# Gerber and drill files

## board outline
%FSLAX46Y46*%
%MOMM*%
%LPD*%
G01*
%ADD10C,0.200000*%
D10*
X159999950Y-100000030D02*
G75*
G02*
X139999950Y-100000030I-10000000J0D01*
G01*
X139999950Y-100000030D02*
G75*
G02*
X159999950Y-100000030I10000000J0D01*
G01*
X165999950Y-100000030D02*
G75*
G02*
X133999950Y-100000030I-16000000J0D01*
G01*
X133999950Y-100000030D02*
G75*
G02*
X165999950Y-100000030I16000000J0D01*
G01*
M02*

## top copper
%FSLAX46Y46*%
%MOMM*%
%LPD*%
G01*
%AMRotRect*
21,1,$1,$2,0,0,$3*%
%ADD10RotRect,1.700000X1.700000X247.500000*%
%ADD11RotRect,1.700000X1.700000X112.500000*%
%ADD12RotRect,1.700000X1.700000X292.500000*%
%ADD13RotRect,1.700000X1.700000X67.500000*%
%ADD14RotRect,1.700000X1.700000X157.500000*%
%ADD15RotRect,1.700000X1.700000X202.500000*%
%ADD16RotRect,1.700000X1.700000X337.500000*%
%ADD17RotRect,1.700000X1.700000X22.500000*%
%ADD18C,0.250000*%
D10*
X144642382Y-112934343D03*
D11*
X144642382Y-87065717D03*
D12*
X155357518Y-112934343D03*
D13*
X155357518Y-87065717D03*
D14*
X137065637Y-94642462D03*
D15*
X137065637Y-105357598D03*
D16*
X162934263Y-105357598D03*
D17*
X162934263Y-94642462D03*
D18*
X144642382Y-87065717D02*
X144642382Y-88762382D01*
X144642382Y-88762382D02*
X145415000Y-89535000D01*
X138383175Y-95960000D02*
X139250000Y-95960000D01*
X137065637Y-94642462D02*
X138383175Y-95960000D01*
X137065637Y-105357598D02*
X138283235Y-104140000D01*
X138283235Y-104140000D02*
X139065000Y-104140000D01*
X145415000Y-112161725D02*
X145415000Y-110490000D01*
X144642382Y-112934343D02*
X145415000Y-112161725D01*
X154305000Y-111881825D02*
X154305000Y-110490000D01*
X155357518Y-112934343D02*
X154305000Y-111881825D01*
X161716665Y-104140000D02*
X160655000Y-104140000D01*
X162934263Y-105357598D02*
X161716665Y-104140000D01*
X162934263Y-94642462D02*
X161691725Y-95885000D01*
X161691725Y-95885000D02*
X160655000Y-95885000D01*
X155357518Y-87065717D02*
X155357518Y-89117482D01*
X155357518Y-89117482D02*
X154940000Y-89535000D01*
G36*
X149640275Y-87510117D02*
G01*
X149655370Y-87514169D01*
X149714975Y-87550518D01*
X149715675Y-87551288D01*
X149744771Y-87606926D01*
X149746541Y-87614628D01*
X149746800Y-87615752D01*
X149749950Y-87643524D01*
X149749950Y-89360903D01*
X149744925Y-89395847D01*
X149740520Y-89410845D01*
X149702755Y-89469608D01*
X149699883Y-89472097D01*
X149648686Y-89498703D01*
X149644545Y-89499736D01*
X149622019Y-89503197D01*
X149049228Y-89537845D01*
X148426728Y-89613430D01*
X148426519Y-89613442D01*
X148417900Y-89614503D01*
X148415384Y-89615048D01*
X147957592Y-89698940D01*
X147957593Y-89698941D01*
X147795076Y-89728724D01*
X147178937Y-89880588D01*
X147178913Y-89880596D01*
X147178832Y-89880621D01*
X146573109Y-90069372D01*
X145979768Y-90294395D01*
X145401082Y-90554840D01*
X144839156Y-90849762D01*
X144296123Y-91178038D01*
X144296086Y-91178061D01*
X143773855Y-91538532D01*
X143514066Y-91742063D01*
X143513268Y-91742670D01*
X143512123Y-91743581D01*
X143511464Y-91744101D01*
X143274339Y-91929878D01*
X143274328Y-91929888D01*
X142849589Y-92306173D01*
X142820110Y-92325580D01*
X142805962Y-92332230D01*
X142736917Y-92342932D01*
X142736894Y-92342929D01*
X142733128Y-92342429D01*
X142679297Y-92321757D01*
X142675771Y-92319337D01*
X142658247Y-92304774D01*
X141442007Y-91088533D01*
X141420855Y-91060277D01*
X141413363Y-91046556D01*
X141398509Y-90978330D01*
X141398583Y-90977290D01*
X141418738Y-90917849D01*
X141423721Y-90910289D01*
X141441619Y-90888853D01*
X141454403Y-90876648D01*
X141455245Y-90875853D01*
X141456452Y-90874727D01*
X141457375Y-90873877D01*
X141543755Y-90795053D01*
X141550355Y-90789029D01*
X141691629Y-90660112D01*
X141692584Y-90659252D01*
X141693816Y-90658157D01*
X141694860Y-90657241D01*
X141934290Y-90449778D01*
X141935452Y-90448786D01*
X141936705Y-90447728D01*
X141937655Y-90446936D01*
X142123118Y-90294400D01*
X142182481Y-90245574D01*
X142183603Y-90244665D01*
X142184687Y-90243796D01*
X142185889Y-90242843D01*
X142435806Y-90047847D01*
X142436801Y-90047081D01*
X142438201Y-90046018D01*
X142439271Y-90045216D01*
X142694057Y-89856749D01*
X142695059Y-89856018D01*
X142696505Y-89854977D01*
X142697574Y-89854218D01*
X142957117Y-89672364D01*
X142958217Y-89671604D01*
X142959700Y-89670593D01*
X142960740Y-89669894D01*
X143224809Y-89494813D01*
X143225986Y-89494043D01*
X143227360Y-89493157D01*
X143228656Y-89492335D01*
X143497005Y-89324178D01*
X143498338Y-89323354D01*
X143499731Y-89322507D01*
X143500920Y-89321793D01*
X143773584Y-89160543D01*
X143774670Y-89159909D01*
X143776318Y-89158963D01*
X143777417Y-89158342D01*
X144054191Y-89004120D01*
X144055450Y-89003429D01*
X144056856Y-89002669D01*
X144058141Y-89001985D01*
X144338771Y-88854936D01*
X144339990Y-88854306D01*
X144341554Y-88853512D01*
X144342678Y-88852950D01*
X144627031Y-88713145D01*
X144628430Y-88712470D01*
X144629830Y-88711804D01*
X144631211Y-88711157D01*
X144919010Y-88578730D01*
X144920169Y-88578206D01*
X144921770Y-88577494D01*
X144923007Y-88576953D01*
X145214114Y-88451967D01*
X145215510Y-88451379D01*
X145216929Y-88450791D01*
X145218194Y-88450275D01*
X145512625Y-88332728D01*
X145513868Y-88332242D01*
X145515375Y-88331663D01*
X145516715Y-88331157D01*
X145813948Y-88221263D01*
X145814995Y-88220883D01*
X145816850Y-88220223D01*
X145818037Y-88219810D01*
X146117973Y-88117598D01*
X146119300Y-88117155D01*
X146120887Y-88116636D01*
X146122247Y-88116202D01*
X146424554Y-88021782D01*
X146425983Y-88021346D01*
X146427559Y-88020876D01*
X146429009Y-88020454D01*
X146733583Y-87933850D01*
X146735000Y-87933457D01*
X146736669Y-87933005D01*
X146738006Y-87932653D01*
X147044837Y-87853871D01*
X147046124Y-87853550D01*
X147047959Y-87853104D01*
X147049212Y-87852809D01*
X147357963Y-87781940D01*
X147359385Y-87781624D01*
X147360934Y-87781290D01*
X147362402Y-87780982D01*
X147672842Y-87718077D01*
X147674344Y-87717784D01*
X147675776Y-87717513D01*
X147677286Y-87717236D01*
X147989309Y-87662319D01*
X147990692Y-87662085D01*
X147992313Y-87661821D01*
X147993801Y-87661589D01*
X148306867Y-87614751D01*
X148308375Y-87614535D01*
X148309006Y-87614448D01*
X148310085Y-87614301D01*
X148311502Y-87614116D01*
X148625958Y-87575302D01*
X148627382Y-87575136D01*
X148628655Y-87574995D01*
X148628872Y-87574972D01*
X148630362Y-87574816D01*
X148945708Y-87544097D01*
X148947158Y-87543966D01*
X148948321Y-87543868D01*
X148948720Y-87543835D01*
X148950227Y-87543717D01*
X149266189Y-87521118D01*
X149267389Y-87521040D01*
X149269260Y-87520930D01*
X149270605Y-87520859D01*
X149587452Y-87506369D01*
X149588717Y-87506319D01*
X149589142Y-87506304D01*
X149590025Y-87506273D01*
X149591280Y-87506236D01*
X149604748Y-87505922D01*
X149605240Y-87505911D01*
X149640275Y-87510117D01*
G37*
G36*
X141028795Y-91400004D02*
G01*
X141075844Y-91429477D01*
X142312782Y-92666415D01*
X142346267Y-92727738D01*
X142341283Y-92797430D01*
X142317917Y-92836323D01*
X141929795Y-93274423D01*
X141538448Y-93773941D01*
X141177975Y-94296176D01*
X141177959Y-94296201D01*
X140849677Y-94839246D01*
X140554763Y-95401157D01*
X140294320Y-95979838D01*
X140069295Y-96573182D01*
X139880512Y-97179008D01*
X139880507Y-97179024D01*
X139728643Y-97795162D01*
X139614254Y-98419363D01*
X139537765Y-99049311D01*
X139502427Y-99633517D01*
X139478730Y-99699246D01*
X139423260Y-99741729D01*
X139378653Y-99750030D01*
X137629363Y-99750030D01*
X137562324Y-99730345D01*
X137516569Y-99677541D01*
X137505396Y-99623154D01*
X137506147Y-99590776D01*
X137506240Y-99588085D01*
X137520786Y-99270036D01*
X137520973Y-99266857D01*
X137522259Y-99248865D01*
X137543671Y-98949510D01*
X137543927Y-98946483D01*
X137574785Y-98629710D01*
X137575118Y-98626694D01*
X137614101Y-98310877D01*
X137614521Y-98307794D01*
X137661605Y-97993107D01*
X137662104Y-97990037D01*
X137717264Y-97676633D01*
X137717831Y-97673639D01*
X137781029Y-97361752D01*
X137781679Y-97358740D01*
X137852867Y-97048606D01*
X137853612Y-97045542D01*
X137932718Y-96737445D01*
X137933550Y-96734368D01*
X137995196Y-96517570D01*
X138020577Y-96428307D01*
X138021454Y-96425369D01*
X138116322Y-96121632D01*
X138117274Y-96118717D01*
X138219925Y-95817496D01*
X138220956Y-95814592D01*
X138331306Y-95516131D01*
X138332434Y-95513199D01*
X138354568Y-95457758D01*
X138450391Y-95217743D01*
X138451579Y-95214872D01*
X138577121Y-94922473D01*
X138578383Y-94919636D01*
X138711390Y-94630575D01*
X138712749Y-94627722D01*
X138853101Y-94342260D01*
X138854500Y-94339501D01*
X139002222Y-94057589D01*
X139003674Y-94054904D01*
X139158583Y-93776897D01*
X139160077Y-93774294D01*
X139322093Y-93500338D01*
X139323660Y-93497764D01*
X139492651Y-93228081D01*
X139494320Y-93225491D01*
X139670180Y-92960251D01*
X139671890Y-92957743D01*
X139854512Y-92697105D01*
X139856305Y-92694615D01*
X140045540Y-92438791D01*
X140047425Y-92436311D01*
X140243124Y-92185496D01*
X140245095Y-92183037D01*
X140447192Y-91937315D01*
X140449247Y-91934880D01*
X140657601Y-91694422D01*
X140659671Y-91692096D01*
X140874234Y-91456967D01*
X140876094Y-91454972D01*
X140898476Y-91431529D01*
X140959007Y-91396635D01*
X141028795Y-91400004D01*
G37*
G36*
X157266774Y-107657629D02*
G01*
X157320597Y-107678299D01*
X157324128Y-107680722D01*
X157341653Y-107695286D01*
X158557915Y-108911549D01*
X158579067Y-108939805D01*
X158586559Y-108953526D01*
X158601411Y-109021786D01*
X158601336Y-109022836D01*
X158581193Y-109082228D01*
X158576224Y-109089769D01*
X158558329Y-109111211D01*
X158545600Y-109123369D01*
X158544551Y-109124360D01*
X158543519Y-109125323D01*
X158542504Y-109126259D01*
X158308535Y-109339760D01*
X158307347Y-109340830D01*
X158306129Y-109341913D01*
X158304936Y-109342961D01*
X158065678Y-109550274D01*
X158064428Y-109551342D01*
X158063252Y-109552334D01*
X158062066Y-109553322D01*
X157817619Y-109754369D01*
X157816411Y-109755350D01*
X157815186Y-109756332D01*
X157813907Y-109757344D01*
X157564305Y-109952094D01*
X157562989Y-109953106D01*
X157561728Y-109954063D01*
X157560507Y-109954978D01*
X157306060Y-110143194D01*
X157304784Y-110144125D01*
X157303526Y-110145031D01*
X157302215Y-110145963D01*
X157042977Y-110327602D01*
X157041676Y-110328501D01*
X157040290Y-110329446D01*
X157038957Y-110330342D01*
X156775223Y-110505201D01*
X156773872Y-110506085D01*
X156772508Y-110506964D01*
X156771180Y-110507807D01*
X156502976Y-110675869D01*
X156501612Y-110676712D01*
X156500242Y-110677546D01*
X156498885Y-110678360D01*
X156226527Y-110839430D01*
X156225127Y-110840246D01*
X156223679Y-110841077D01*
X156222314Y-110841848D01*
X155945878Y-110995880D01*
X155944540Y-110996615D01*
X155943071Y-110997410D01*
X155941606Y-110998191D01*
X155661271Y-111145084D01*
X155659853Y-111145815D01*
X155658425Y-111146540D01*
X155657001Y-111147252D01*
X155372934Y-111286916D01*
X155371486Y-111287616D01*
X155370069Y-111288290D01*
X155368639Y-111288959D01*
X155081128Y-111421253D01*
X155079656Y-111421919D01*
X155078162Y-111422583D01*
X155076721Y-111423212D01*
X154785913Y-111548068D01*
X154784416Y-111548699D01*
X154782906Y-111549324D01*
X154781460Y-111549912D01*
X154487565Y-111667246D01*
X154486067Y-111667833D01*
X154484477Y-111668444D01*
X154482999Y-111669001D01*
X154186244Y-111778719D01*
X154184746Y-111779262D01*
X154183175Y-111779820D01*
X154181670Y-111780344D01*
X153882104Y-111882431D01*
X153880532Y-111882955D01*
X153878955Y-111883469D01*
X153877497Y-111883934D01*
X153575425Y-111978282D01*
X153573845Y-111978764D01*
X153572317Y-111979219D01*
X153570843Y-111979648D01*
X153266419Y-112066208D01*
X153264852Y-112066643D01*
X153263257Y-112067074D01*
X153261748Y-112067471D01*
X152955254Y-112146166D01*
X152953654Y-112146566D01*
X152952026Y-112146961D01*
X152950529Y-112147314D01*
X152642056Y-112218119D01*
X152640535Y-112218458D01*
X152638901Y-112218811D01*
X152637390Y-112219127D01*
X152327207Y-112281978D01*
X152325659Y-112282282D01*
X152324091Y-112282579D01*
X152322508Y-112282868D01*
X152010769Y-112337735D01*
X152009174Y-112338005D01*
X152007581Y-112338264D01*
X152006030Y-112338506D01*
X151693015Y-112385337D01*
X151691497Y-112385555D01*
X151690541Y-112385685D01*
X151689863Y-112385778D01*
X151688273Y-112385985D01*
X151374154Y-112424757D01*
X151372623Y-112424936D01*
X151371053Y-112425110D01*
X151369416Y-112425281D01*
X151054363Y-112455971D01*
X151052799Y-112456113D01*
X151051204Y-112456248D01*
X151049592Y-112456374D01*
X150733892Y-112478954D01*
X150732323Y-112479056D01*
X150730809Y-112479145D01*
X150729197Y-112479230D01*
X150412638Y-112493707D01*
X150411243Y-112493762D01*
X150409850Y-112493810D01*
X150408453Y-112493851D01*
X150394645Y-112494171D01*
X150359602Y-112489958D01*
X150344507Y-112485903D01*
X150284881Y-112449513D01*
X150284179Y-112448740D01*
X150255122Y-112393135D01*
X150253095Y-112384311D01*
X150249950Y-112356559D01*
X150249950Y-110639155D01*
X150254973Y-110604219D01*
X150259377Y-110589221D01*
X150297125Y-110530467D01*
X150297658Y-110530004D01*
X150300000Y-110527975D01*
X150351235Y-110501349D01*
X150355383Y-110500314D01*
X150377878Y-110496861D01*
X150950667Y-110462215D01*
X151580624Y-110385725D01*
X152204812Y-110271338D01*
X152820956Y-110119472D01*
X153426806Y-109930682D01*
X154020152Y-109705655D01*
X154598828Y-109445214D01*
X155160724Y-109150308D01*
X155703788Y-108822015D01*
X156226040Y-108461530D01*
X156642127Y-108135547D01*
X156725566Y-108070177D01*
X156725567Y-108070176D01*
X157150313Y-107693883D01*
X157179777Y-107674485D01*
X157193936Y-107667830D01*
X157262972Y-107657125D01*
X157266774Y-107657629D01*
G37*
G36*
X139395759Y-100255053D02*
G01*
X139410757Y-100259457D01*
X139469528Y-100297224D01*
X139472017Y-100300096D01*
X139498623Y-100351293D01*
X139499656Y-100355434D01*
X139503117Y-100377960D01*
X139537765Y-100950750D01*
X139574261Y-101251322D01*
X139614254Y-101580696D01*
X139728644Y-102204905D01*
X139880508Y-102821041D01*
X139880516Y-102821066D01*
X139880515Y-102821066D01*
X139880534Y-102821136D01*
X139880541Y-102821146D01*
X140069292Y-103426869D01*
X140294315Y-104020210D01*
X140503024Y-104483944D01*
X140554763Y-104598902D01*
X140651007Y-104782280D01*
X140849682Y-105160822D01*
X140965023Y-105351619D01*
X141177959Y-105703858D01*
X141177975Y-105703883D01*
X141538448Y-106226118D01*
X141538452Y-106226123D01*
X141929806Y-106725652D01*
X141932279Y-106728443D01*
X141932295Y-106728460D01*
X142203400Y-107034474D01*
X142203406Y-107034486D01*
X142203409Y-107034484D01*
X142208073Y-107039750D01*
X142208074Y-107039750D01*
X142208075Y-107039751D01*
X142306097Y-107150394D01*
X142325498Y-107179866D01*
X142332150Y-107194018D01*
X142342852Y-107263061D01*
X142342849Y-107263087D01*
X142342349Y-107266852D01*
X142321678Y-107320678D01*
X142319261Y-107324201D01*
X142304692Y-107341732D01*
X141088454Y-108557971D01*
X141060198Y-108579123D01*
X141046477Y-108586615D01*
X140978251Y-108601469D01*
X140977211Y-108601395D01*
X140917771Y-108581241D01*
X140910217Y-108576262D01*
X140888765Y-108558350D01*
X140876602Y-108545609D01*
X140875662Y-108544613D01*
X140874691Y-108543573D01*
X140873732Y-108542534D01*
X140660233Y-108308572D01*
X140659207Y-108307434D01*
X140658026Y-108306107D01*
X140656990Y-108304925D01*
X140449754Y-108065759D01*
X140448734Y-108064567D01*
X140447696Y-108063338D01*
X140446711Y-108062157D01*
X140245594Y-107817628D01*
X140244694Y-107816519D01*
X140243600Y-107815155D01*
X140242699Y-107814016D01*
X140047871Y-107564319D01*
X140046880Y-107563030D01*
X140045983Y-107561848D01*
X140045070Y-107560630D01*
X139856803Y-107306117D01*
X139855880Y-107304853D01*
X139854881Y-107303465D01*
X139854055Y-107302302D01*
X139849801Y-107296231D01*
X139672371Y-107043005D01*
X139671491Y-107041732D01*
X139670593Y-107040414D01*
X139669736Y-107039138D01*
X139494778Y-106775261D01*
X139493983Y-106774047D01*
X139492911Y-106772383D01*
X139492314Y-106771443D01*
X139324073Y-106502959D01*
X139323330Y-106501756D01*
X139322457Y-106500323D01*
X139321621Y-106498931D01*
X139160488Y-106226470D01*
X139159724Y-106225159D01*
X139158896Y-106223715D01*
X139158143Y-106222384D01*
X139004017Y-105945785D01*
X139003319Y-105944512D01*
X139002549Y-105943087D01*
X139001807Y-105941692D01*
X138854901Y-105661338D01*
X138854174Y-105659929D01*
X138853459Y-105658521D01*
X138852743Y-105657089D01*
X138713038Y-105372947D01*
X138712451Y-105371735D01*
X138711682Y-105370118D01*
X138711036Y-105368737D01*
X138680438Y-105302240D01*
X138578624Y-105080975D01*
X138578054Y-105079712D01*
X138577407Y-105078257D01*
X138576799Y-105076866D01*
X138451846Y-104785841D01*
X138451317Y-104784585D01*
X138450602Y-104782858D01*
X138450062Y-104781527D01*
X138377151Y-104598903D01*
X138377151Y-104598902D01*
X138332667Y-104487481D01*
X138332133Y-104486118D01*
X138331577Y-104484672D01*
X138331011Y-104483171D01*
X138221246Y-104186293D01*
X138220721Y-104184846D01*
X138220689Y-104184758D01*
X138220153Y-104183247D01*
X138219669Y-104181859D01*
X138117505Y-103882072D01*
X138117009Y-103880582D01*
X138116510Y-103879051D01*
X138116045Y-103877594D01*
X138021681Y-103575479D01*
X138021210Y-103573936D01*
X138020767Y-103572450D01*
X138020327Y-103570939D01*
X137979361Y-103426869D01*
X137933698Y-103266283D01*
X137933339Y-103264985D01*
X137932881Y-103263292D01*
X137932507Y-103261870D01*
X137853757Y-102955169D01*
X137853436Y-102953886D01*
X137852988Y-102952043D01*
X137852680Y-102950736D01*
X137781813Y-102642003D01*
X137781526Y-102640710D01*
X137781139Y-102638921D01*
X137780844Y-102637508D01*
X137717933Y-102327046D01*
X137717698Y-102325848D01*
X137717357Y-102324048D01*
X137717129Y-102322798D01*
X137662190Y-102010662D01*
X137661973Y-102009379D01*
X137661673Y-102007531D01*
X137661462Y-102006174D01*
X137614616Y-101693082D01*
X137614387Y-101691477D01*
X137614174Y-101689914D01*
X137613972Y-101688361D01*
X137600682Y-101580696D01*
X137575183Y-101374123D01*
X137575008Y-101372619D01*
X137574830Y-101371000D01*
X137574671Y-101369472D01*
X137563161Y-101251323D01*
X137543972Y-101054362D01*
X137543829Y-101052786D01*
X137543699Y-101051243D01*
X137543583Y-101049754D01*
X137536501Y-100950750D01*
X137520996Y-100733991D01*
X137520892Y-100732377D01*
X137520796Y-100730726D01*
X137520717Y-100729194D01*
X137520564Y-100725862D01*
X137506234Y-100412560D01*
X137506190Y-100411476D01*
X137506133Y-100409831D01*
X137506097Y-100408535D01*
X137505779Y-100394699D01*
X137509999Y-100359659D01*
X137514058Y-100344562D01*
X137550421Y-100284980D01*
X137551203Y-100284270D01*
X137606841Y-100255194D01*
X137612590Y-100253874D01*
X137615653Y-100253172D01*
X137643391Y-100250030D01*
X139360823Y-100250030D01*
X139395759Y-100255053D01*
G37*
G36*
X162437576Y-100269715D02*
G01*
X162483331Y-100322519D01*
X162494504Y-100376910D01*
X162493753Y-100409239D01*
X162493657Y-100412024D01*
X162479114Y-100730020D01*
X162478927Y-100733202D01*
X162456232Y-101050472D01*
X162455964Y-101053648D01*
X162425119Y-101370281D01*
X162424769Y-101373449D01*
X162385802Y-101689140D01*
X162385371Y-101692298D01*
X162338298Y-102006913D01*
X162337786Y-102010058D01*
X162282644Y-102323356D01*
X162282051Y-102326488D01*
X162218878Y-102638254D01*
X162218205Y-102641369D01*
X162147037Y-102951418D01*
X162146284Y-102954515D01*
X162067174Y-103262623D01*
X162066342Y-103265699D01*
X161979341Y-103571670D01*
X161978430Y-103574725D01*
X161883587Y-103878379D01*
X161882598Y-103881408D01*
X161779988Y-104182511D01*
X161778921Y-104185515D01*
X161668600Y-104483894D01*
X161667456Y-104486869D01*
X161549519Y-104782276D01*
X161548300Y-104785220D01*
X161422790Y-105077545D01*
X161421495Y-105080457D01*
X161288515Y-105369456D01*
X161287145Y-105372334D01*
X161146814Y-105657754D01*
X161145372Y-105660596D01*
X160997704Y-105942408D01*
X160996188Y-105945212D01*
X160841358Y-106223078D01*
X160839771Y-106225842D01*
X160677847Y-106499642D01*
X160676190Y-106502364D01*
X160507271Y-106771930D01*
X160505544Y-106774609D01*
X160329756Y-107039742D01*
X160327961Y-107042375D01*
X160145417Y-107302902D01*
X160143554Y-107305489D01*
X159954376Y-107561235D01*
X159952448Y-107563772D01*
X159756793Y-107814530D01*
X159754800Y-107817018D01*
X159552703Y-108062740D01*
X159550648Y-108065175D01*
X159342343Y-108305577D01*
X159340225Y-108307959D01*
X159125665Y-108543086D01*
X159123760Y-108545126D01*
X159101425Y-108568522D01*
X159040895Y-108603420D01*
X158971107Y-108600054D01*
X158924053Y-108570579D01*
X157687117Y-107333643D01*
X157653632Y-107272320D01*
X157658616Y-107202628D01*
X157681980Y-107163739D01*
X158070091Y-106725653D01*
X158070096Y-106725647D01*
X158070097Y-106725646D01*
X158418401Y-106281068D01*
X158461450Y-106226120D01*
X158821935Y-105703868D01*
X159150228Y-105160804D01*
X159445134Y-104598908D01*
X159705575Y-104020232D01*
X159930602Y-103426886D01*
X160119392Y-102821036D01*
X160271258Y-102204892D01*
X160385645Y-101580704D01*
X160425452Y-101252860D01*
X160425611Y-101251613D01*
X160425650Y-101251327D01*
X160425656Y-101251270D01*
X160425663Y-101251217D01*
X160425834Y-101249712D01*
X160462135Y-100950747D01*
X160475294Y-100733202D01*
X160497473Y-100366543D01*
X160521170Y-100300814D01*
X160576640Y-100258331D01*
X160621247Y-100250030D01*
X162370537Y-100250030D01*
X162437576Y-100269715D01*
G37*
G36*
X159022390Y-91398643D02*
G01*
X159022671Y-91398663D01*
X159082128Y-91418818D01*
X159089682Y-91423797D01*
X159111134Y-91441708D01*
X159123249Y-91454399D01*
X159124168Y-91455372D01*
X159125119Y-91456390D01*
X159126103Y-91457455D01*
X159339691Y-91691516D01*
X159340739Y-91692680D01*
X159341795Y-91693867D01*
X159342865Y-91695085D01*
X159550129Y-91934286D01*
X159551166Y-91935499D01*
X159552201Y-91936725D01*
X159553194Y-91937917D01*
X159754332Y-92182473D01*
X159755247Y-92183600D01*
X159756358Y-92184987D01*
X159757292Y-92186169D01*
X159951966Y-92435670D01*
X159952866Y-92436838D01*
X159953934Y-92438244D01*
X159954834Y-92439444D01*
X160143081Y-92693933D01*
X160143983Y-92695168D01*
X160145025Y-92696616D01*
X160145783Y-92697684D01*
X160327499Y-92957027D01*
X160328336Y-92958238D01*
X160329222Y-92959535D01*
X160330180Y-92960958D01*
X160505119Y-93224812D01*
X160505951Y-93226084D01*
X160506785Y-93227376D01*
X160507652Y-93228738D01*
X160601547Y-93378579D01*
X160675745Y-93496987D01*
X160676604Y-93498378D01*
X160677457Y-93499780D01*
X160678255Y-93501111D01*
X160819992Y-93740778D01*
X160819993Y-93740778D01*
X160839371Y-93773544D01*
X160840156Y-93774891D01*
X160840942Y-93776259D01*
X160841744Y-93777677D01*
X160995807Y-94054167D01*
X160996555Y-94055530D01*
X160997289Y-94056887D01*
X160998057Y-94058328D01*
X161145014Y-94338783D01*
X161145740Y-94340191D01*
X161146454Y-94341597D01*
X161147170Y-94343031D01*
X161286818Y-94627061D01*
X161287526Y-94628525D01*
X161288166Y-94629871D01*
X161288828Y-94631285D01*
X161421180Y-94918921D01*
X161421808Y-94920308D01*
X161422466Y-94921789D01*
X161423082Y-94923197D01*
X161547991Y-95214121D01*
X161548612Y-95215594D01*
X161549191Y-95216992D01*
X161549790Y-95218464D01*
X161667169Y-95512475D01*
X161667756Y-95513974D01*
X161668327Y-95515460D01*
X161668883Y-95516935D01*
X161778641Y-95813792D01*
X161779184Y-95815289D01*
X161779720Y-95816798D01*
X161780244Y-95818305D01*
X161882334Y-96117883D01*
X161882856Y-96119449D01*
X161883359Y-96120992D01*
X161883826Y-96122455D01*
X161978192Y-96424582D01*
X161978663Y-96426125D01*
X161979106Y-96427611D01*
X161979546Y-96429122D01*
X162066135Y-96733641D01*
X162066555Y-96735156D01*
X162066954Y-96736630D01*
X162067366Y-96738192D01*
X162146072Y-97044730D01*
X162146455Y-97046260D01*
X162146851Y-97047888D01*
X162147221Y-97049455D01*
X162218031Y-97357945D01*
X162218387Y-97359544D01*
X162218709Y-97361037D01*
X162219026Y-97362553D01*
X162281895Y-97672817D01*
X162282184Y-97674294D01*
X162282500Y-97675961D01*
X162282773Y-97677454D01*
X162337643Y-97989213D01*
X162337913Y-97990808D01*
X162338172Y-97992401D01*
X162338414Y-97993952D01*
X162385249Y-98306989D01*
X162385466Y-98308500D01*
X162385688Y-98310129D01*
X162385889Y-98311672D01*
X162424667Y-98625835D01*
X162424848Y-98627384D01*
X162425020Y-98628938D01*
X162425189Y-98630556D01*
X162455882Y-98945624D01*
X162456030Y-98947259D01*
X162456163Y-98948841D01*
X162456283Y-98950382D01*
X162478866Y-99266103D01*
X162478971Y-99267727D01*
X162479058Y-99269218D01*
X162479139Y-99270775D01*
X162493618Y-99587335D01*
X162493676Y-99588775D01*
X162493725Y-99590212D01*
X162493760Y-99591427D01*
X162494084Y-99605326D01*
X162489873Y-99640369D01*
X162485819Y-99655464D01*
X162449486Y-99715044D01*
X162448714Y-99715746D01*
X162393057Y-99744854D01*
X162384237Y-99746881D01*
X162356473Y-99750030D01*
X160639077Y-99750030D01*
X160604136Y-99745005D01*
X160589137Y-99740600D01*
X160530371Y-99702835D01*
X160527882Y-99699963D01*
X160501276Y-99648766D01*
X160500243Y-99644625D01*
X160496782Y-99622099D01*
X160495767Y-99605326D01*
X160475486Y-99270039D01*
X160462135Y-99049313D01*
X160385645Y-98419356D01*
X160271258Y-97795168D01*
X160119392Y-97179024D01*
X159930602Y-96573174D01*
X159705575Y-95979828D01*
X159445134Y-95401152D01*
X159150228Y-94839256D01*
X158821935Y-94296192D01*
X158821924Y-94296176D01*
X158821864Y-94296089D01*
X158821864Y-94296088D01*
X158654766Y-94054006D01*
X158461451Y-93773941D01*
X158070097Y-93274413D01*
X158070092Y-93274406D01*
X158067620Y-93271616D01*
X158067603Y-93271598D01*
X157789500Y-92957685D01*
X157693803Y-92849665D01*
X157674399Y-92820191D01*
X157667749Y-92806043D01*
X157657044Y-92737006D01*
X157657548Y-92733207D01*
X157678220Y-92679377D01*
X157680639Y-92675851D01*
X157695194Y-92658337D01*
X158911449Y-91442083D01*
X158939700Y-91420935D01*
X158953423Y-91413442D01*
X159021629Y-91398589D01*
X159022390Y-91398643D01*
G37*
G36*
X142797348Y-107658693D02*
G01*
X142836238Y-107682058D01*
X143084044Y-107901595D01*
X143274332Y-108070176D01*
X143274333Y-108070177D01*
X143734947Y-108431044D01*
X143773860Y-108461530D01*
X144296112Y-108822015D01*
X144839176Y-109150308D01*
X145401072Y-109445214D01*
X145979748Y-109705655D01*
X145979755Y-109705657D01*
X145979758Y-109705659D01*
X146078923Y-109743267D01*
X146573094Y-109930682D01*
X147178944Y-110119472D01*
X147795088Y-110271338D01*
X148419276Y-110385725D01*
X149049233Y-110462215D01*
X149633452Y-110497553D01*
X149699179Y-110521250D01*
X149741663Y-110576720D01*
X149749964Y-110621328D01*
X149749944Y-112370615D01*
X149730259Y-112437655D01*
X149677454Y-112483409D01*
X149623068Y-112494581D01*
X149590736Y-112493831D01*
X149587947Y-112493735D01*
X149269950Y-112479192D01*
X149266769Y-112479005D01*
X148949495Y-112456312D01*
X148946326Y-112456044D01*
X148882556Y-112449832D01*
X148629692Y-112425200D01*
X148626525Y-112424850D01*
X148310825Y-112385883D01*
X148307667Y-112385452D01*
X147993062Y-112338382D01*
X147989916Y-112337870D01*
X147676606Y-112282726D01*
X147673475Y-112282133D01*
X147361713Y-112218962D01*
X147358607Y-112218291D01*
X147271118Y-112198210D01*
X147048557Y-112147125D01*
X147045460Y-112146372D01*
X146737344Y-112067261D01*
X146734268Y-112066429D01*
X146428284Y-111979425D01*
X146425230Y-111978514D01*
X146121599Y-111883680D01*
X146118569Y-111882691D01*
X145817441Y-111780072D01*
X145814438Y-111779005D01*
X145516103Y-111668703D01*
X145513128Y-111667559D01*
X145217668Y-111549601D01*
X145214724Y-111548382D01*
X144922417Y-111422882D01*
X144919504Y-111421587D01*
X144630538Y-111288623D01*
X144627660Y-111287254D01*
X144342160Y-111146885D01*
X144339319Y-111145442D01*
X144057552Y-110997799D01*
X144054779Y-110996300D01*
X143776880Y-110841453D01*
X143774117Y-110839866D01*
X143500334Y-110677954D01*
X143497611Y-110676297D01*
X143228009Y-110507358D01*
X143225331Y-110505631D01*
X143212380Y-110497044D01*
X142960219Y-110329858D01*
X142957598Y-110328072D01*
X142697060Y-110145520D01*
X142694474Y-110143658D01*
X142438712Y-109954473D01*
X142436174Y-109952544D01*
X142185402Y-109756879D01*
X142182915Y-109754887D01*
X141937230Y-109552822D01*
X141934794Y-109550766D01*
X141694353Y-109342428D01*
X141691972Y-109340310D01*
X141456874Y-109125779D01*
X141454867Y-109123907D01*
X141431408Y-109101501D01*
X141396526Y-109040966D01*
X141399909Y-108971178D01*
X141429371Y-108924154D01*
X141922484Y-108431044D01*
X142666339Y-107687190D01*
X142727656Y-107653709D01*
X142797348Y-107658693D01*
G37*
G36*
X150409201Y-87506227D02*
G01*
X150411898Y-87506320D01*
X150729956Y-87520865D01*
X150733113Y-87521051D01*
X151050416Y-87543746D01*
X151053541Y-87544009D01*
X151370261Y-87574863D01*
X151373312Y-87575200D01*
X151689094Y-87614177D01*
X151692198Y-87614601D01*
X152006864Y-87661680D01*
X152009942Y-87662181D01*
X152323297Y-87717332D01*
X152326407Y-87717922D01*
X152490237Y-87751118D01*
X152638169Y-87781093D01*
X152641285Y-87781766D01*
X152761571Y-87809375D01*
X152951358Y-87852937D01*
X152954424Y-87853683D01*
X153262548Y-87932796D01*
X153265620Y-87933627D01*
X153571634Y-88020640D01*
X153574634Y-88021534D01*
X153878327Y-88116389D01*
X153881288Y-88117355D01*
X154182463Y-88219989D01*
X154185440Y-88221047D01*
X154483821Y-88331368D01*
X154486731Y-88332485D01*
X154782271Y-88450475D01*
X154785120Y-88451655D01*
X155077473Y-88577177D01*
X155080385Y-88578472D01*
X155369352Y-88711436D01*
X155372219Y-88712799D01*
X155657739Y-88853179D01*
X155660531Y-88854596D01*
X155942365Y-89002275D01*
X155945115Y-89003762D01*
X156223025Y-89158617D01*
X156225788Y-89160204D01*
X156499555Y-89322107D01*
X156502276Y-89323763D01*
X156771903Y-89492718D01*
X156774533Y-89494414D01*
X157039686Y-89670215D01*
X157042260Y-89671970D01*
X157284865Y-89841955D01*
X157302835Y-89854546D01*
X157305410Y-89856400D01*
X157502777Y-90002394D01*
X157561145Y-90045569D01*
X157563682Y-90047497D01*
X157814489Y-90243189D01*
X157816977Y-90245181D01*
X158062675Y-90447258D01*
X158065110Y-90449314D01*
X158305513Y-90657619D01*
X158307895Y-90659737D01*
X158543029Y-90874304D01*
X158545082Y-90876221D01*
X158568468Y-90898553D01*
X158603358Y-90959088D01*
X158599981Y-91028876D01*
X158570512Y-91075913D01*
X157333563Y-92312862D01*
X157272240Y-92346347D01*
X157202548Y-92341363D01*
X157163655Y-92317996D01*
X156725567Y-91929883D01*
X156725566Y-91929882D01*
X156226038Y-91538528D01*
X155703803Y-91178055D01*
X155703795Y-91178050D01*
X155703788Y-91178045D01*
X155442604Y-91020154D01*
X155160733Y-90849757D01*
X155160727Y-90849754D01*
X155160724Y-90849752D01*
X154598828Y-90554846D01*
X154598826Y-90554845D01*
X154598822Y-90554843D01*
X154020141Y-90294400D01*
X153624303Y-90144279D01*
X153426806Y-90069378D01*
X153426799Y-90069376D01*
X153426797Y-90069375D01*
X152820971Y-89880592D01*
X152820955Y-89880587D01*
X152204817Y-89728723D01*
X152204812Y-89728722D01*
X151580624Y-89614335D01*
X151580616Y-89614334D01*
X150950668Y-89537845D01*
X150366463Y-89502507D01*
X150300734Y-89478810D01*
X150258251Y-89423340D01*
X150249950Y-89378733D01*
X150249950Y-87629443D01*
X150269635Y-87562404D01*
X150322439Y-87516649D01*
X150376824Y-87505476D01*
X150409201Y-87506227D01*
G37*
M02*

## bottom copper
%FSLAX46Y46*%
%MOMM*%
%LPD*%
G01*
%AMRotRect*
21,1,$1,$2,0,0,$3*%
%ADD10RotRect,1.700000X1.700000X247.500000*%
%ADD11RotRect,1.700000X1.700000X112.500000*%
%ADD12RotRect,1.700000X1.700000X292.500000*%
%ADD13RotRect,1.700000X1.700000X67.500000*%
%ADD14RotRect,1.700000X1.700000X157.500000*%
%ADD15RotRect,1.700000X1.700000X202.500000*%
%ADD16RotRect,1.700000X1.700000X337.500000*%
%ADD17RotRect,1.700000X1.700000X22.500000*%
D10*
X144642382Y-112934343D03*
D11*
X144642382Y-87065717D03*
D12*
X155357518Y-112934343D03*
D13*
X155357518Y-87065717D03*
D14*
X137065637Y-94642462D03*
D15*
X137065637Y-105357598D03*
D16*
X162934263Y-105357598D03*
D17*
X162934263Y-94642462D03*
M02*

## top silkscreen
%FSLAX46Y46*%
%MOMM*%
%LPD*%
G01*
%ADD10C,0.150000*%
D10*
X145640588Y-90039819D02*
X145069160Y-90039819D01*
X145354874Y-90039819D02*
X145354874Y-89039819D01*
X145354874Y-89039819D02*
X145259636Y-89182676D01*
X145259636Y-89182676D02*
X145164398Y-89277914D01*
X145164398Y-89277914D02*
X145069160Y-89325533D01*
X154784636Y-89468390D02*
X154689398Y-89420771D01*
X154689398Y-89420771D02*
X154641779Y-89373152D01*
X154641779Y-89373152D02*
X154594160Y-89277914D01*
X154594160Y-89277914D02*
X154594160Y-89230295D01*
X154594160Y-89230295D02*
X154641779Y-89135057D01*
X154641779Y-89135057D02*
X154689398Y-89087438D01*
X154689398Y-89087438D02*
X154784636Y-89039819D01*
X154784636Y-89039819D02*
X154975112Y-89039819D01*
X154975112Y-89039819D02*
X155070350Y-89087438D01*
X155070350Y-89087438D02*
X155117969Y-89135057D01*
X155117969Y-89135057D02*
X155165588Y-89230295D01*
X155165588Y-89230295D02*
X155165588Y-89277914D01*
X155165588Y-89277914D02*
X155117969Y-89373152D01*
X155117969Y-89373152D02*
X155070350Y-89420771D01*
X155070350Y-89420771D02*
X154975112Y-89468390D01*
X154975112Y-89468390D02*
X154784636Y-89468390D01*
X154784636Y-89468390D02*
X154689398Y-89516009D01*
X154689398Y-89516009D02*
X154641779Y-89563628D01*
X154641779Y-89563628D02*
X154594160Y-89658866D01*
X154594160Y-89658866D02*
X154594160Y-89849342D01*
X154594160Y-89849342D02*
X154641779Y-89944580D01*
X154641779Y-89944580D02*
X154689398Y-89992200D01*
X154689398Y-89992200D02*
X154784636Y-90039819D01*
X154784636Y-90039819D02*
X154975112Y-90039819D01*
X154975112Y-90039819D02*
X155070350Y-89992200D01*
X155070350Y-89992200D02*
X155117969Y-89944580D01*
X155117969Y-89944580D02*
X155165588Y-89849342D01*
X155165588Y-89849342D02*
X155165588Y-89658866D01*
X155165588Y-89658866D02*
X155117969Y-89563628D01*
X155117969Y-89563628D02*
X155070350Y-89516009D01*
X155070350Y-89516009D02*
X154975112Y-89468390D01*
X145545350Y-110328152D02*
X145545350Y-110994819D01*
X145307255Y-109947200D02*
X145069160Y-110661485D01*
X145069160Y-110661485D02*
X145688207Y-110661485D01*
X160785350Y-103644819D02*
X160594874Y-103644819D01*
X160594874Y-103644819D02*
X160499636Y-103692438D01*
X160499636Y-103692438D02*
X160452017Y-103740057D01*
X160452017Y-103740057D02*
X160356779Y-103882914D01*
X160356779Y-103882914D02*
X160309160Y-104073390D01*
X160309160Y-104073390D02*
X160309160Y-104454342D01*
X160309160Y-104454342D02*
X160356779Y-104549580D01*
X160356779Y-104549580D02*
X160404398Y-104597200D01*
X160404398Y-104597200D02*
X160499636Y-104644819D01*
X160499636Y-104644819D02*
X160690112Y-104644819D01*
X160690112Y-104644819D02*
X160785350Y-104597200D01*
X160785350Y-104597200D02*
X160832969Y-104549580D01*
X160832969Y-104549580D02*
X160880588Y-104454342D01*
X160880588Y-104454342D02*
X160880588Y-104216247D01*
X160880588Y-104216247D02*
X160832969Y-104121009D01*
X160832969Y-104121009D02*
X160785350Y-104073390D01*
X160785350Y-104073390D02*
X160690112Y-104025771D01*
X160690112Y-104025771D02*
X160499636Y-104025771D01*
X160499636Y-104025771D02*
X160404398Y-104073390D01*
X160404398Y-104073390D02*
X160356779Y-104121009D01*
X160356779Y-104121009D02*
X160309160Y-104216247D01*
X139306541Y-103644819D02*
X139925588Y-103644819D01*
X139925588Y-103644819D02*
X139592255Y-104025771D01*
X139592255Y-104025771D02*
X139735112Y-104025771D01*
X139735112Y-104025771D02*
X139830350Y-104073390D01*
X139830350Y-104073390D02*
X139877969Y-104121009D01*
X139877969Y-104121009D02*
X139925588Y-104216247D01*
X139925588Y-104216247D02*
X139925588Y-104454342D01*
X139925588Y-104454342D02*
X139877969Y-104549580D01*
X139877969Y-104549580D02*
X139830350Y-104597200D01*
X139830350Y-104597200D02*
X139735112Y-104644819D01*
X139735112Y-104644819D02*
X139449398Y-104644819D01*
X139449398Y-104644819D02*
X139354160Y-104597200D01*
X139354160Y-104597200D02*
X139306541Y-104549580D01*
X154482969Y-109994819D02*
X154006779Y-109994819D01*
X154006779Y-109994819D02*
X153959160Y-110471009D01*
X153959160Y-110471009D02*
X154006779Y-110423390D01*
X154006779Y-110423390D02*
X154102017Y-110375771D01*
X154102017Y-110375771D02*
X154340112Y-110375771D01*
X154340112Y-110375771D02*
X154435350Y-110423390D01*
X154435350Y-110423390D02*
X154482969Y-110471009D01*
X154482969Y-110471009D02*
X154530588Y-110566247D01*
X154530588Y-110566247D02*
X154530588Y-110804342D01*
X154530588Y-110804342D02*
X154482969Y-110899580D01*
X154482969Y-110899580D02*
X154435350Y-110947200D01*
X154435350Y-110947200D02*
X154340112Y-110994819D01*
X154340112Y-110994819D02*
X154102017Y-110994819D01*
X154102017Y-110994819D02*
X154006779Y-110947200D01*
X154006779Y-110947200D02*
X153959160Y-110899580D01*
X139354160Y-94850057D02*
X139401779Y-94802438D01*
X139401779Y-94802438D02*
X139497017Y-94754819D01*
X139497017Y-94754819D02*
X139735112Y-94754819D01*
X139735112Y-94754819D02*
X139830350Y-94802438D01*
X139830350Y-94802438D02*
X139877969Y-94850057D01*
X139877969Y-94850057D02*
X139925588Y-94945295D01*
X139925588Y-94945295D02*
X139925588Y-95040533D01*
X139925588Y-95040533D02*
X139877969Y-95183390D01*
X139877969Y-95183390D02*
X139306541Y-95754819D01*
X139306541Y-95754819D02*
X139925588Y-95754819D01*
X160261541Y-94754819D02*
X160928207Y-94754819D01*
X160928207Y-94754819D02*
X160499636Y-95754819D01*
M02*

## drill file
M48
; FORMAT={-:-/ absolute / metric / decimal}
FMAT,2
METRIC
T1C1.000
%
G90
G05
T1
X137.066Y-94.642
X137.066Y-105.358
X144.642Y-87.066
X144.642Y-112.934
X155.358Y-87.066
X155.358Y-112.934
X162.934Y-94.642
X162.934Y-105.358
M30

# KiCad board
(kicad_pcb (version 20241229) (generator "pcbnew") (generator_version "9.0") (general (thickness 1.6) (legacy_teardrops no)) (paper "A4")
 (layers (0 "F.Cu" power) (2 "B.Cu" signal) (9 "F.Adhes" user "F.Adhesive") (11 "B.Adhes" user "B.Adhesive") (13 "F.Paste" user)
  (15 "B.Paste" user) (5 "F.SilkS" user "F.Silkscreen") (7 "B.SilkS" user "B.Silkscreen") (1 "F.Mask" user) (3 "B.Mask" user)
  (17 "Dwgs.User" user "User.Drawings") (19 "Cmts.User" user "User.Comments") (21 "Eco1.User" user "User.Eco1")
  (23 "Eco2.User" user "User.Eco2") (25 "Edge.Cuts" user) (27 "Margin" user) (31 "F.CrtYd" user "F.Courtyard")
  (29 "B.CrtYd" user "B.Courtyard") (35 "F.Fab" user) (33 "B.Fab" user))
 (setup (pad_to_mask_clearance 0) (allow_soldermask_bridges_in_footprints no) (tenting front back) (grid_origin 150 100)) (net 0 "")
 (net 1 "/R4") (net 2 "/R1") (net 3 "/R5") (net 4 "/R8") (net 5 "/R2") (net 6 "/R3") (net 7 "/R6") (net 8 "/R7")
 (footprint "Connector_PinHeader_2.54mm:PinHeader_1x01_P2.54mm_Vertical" (layer "B.Cu") (at 144.642382 112.934343 -112.5)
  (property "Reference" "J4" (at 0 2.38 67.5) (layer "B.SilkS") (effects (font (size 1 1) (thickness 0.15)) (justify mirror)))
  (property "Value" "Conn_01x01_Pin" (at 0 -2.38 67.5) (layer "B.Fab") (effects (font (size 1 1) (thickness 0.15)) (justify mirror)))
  (pad "1" thru_hole rect (at 0 0 247.5) (size 1.7 1.7) (drill 1) (layers "*.Cu" "*.Mask") (remove_unused_layers no) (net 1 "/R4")))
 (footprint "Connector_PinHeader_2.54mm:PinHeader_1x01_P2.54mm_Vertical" (layer "B.Cu") (at 144.642382 87.06571700000001 112.5)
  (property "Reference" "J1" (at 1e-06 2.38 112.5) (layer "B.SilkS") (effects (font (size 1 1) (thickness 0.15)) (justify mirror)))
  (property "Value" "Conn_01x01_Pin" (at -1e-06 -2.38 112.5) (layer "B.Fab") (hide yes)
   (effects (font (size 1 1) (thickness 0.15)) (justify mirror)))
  (pad "1" thru_hole rect (at 0 0 112.5) (size 1.7 1.7) (drill 1) (layers "*.Cu" "*.Mask") (remove_unused_layers no) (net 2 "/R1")))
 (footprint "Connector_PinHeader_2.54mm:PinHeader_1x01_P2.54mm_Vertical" (layer "B.Cu") (at 155.357518 112.934343 -67.5)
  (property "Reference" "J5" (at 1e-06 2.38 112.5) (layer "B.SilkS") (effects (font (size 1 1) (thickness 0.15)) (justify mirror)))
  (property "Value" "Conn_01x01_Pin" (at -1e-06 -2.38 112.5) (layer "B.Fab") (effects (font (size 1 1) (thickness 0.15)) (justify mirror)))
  (pad "1" thru_hole rect (at 0 0 292.5) (size 1.7 1.7) (drill 1) (layers "*.Cu" "*.Mask") (remove_unused_layers no) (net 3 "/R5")))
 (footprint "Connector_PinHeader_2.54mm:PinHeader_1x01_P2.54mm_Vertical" (layer "B.Cu") (at 155.357518 87.06571700000001 67.5)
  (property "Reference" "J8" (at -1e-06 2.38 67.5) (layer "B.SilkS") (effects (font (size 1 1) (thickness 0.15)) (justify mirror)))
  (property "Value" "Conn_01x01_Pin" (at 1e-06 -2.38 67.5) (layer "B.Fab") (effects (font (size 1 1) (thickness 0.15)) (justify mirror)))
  (pad "1" thru_hole rect (at 0 0 67.5) (size 1.7 1.7) (drill 1) (layers "*.Cu" "*.Mask") (remove_unused_layers no) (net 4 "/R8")))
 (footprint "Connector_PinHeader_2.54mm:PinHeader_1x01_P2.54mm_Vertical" (layer "B.Cu") (at 137.065637 94.64246199999999 157.5)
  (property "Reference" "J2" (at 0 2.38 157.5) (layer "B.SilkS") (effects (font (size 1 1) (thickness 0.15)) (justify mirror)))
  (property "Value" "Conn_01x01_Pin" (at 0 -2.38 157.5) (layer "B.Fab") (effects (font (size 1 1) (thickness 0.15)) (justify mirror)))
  (pad "1" thru_hole rect (at 0 0 157.5) (size 1.7 1.7) (drill 1) (layers "*.Cu" "*.Mask") (remove_unused_layers no) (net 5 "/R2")))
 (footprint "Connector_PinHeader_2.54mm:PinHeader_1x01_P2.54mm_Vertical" (layer "B.Cu") (at 137.065637 105.357598 -157.5)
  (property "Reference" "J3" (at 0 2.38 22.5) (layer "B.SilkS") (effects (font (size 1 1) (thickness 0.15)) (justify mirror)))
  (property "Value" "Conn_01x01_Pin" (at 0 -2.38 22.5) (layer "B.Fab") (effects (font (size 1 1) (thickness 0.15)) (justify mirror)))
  (pad "1" thru_hole rect (at 0 0 202.5) (size 1.7 1.7) (drill 1) (layers "*.Cu" "*.Mask") (remove_unused_layers no) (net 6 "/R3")))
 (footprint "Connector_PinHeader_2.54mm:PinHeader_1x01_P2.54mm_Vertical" (layer "B.Cu") (at 162.934263 105.357598 -22.5)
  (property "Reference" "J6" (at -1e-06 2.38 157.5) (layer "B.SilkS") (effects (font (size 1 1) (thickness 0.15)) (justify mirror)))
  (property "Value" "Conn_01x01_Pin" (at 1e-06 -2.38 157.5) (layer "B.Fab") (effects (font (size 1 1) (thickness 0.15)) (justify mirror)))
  (pad "1" thru_hole rect (at 0 0 337.5) (size 1.7 1.7) (drill 1) (layers "*.Cu" "*.Mask") (remove_unused_layers no) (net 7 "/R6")))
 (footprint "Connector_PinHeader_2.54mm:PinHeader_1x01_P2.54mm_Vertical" (layer "B.Cu") (at 162.934263 94.64246199999999 22.5)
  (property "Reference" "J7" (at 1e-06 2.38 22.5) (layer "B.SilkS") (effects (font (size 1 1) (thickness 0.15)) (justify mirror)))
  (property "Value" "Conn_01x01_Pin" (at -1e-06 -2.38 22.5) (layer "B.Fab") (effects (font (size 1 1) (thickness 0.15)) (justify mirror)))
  (pad "1" thru_hole rect (at 0 0 22.5) (size 1.7 1.7) (drill 1) (layers "*.Cu" "*.Mask") (remove_unused_layers no) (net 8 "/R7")))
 (gr_circle (center 149.99995 100.00003) (end 159.99995 100.00003) (stroke (width 0.2) (type solid)) (fill no) (layer "Edge.Cuts"))
 (gr_circle (center 149.99995 100.00003) (end 165.99995 100.00003) (stroke (width 0.2) (type solid)) (fill no) (layer "Edge.Cuts"))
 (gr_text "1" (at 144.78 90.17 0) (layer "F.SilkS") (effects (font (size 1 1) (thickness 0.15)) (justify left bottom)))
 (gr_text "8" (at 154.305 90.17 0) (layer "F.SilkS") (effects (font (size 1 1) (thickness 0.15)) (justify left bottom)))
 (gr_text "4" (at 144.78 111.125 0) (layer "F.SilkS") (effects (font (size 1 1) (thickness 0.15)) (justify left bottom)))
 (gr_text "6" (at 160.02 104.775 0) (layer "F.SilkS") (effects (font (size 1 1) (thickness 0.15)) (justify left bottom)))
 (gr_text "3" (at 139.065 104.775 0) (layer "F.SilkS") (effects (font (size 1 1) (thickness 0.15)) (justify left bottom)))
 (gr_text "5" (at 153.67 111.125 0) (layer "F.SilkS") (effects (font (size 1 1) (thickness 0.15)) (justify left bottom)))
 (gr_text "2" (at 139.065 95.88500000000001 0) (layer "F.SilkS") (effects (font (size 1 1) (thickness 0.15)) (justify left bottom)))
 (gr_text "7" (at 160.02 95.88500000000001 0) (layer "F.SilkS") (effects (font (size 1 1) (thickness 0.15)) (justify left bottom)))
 (segment (start 144.642382 87.06571700000001) (end 144.642382 88.762382) (width 0.25) (layer "F.Cu") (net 2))
 (segment (start 144.642382 88.762382) (end 145.415 89.535) (width 0.25) (layer "F.Cu") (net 2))
 (segment (start 138.383175 95.95999999999999) (end 139.25 95.95999999999999) (width 0.25) (layer "F.Cu") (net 5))
 (segment (start 137.065637 94.64246199999999) (end 138.383175 95.95999999999999) (width 0.25) (layer "F.Cu") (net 5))
 (segment (start 137.065637 105.357598) (end 138.283235 104.14) (width 0.25) (layer "F.Cu") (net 6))
 (segment (start 138.283235 104.14) (end 139.065 104.14) (width 0.25) (layer "F.Cu") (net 6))
 (segment (start 145.415 112.161725) (end 145.415 110.49) (width 0.25) (layer "F.Cu") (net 1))
 (segment (start 144.642382 112.934343) (end 145.415 112.161725) (width 0.25) (layer "F.Cu") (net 1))
 (segment (start 154.305 111.881825) (end 154.305 110.49) (width 0.25) (layer "F.Cu") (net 3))
 (segment (start 155.357518 112.934343) (end 154.305 111.881825) (width 0.25) (layer "F.Cu") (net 3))
 (segment (start 161.716665 104.14) (end 160.655 104.14) (width 0.25) (layer "F.Cu") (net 7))
 (segment (start 162.934263 105.357598) (end 161.716665 104.14) (width 0.25) (layer "F.Cu") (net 7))
 (segment (start 162.934263 94.64246199999999) (end 161.691725 95.88500000000001) (width 0.25) (layer "F.Cu") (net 8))
 (segment (start 161.691725 95.88500000000001) (end 160.655 95.88500000000001) (width 0.25) (layer "F.Cu") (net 8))
 (segment (start 155.357518 87.06571700000001) (end 155.357518 89.117482) (width 0.25) (layer "F.Cu") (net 4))
 (segment (start 155.357518 89.117482) (end 154.94 89.535) (width 0.25) (layer "F.Cu") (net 4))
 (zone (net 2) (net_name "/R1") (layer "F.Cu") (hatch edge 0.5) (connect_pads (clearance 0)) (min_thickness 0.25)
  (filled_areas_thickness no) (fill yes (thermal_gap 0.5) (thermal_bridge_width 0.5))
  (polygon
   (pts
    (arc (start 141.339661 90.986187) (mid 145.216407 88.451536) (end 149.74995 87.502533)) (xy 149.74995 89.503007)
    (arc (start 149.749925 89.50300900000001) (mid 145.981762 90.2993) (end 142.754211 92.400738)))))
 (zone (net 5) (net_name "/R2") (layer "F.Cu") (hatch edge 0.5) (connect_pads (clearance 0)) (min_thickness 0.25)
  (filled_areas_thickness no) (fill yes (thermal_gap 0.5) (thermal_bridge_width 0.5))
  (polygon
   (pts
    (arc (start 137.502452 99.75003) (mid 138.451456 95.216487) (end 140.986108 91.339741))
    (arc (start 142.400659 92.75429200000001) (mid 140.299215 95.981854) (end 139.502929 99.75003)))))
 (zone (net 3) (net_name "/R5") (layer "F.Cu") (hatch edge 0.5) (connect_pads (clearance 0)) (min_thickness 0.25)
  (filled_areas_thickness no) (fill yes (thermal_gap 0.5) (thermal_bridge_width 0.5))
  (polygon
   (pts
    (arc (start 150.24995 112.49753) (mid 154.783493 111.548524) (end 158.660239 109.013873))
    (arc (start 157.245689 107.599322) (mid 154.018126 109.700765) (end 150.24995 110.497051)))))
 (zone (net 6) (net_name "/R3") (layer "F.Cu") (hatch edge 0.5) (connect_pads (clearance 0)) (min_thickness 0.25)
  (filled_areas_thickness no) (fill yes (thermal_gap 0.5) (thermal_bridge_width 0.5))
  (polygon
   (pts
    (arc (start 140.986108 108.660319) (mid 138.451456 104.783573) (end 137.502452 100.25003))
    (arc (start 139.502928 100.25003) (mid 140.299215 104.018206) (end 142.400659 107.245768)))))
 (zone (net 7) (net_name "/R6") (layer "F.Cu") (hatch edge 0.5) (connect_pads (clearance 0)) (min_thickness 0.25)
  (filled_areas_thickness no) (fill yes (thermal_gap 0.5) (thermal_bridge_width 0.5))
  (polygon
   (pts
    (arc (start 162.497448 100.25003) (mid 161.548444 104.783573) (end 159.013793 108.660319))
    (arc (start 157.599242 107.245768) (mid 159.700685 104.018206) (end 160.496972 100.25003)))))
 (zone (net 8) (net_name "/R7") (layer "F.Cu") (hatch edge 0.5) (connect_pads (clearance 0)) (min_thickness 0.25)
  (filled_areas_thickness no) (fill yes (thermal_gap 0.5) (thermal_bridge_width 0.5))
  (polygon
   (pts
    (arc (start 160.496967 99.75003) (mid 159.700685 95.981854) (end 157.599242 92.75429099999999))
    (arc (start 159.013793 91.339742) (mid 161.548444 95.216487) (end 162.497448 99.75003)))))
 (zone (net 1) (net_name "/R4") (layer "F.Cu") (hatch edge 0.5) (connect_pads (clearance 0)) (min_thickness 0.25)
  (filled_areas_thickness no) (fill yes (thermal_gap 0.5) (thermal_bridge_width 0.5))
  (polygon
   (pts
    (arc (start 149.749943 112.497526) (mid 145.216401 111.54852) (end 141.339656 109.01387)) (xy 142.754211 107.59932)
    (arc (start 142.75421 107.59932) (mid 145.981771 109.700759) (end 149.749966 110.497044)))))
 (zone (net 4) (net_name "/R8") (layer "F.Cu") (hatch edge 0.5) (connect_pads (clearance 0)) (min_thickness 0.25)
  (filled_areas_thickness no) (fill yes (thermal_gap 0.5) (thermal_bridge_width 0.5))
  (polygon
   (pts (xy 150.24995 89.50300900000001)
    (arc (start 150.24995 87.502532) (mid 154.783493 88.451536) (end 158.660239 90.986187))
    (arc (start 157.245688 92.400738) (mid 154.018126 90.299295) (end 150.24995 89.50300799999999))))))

